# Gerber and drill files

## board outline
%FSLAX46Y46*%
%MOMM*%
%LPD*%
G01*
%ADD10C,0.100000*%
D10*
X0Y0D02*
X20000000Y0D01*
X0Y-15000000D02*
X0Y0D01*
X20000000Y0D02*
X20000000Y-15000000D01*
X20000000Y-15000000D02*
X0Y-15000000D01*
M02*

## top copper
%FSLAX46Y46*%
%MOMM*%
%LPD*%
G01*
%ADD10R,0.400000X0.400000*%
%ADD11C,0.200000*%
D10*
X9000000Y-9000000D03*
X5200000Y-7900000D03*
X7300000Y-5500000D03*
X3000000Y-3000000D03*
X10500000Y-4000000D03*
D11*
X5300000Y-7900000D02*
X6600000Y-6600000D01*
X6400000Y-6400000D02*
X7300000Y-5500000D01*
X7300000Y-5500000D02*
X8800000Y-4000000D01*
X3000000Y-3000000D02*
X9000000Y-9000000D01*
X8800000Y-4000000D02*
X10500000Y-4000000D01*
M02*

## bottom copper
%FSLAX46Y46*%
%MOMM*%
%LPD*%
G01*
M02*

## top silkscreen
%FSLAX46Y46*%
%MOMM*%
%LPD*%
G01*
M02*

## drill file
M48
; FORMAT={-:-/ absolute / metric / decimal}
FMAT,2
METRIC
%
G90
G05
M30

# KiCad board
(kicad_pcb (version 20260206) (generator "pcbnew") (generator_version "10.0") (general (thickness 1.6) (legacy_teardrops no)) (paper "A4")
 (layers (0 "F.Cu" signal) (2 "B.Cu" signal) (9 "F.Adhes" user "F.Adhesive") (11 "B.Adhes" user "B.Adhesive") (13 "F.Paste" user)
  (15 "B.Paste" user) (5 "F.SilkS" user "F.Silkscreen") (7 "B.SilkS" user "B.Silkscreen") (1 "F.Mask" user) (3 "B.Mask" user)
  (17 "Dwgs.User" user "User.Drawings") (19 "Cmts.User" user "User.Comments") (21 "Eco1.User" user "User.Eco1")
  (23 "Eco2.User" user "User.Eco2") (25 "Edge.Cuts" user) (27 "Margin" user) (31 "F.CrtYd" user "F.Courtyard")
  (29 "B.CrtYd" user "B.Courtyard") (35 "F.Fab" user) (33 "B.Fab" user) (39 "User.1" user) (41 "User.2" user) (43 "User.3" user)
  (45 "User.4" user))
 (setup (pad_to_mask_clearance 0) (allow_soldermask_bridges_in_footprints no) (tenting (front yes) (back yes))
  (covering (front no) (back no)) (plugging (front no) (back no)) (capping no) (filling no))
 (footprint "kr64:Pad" (layer "F.Cu") (at 9 9)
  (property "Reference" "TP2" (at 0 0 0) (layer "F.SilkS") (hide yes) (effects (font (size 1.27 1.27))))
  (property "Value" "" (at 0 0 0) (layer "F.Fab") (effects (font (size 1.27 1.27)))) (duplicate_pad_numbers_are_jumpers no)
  (pad "1" smd rect (at 0 0) (size 0.4 0.4) (layers "F.Cu" "F.Mask" "F.Paste") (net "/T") (thermal_bridge_angle 45)))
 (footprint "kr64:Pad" (layer "F.Cu") (at 5.2 7.9)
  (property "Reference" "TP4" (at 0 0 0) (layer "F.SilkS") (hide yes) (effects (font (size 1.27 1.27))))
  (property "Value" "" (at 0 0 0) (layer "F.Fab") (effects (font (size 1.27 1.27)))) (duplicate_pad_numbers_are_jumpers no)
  (pad "1" smd rect (at 0 0) (size 0.4 0.4) (layers "F.Cu" "F.Mask" "F.Paste") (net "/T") (thermal_bridge_angle 45)))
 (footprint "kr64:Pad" (layer "F.Cu") (at 7.3 5.5)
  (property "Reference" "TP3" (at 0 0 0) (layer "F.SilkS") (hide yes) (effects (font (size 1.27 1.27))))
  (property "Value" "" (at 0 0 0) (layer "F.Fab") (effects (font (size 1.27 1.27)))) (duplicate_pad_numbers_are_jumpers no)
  (pad "1" smd rect (at 0 0) (size 0.4 0.4) (layers "F.Cu" "F.Mask" "F.Paste") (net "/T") (thermal_bridge_angle 45)))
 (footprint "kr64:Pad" (layer "F.Cu") (at 3 3)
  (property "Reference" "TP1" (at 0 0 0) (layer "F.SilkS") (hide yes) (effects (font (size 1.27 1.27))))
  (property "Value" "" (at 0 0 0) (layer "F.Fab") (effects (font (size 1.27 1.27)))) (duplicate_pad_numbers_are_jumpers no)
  (pad "1" smd rect (at 0 0) (size 0.4 0.4) (layers "F.Cu" "F.Mask" "F.Paste") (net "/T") (thermal_bridge_angle 45)))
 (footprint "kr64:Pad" (layer "F.Cu") (at 10.5 4)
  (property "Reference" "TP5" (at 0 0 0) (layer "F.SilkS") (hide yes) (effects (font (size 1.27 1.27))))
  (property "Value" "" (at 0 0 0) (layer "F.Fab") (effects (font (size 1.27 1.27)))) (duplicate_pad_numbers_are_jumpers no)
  (pad "1" smd rect (at 0 0) (size 0.4 0.4) (layers "F.Cu" "F.Mask" "F.Paste") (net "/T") (thermal_bridge_angle 45)))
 (gr_line (start 0 0) (end 20 0) (stroke (width 0.1) (type default)) (layer "Edge.Cuts"))
 (gr_line (start 0 15) (end 0 0) (stroke (width 0.1) (type default)) (layer "Edge.Cuts"))
 (gr_line (start 20 0) (end 20 15) (stroke (width 0.1) (type default)) (layer "Edge.Cuts"))
 (gr_line (start 20 15) (end 0 15) (stroke (width 0.1) (type default)) (layer "Edge.Cuts"))
 (segment (start 5.3 7.9) (end 6.6 6.6) (width 0.2) (layer "F.Cu") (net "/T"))
 (segment (start 6.4 6.4) (end 7.3 5.5) (width 0.2) (layer "F.Cu") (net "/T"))
 (segment (start 7.3 5.5) (end 8.8 4) (width 0.2) (layer "F.Cu") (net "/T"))
 (segment (start 3 3) (end 9 9) (width 0.2) (layer "F.Cu") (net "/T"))
 (segment (start 8.8 4) (end 10.5 4) (width 0.2) (layer "F.Cu") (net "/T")))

